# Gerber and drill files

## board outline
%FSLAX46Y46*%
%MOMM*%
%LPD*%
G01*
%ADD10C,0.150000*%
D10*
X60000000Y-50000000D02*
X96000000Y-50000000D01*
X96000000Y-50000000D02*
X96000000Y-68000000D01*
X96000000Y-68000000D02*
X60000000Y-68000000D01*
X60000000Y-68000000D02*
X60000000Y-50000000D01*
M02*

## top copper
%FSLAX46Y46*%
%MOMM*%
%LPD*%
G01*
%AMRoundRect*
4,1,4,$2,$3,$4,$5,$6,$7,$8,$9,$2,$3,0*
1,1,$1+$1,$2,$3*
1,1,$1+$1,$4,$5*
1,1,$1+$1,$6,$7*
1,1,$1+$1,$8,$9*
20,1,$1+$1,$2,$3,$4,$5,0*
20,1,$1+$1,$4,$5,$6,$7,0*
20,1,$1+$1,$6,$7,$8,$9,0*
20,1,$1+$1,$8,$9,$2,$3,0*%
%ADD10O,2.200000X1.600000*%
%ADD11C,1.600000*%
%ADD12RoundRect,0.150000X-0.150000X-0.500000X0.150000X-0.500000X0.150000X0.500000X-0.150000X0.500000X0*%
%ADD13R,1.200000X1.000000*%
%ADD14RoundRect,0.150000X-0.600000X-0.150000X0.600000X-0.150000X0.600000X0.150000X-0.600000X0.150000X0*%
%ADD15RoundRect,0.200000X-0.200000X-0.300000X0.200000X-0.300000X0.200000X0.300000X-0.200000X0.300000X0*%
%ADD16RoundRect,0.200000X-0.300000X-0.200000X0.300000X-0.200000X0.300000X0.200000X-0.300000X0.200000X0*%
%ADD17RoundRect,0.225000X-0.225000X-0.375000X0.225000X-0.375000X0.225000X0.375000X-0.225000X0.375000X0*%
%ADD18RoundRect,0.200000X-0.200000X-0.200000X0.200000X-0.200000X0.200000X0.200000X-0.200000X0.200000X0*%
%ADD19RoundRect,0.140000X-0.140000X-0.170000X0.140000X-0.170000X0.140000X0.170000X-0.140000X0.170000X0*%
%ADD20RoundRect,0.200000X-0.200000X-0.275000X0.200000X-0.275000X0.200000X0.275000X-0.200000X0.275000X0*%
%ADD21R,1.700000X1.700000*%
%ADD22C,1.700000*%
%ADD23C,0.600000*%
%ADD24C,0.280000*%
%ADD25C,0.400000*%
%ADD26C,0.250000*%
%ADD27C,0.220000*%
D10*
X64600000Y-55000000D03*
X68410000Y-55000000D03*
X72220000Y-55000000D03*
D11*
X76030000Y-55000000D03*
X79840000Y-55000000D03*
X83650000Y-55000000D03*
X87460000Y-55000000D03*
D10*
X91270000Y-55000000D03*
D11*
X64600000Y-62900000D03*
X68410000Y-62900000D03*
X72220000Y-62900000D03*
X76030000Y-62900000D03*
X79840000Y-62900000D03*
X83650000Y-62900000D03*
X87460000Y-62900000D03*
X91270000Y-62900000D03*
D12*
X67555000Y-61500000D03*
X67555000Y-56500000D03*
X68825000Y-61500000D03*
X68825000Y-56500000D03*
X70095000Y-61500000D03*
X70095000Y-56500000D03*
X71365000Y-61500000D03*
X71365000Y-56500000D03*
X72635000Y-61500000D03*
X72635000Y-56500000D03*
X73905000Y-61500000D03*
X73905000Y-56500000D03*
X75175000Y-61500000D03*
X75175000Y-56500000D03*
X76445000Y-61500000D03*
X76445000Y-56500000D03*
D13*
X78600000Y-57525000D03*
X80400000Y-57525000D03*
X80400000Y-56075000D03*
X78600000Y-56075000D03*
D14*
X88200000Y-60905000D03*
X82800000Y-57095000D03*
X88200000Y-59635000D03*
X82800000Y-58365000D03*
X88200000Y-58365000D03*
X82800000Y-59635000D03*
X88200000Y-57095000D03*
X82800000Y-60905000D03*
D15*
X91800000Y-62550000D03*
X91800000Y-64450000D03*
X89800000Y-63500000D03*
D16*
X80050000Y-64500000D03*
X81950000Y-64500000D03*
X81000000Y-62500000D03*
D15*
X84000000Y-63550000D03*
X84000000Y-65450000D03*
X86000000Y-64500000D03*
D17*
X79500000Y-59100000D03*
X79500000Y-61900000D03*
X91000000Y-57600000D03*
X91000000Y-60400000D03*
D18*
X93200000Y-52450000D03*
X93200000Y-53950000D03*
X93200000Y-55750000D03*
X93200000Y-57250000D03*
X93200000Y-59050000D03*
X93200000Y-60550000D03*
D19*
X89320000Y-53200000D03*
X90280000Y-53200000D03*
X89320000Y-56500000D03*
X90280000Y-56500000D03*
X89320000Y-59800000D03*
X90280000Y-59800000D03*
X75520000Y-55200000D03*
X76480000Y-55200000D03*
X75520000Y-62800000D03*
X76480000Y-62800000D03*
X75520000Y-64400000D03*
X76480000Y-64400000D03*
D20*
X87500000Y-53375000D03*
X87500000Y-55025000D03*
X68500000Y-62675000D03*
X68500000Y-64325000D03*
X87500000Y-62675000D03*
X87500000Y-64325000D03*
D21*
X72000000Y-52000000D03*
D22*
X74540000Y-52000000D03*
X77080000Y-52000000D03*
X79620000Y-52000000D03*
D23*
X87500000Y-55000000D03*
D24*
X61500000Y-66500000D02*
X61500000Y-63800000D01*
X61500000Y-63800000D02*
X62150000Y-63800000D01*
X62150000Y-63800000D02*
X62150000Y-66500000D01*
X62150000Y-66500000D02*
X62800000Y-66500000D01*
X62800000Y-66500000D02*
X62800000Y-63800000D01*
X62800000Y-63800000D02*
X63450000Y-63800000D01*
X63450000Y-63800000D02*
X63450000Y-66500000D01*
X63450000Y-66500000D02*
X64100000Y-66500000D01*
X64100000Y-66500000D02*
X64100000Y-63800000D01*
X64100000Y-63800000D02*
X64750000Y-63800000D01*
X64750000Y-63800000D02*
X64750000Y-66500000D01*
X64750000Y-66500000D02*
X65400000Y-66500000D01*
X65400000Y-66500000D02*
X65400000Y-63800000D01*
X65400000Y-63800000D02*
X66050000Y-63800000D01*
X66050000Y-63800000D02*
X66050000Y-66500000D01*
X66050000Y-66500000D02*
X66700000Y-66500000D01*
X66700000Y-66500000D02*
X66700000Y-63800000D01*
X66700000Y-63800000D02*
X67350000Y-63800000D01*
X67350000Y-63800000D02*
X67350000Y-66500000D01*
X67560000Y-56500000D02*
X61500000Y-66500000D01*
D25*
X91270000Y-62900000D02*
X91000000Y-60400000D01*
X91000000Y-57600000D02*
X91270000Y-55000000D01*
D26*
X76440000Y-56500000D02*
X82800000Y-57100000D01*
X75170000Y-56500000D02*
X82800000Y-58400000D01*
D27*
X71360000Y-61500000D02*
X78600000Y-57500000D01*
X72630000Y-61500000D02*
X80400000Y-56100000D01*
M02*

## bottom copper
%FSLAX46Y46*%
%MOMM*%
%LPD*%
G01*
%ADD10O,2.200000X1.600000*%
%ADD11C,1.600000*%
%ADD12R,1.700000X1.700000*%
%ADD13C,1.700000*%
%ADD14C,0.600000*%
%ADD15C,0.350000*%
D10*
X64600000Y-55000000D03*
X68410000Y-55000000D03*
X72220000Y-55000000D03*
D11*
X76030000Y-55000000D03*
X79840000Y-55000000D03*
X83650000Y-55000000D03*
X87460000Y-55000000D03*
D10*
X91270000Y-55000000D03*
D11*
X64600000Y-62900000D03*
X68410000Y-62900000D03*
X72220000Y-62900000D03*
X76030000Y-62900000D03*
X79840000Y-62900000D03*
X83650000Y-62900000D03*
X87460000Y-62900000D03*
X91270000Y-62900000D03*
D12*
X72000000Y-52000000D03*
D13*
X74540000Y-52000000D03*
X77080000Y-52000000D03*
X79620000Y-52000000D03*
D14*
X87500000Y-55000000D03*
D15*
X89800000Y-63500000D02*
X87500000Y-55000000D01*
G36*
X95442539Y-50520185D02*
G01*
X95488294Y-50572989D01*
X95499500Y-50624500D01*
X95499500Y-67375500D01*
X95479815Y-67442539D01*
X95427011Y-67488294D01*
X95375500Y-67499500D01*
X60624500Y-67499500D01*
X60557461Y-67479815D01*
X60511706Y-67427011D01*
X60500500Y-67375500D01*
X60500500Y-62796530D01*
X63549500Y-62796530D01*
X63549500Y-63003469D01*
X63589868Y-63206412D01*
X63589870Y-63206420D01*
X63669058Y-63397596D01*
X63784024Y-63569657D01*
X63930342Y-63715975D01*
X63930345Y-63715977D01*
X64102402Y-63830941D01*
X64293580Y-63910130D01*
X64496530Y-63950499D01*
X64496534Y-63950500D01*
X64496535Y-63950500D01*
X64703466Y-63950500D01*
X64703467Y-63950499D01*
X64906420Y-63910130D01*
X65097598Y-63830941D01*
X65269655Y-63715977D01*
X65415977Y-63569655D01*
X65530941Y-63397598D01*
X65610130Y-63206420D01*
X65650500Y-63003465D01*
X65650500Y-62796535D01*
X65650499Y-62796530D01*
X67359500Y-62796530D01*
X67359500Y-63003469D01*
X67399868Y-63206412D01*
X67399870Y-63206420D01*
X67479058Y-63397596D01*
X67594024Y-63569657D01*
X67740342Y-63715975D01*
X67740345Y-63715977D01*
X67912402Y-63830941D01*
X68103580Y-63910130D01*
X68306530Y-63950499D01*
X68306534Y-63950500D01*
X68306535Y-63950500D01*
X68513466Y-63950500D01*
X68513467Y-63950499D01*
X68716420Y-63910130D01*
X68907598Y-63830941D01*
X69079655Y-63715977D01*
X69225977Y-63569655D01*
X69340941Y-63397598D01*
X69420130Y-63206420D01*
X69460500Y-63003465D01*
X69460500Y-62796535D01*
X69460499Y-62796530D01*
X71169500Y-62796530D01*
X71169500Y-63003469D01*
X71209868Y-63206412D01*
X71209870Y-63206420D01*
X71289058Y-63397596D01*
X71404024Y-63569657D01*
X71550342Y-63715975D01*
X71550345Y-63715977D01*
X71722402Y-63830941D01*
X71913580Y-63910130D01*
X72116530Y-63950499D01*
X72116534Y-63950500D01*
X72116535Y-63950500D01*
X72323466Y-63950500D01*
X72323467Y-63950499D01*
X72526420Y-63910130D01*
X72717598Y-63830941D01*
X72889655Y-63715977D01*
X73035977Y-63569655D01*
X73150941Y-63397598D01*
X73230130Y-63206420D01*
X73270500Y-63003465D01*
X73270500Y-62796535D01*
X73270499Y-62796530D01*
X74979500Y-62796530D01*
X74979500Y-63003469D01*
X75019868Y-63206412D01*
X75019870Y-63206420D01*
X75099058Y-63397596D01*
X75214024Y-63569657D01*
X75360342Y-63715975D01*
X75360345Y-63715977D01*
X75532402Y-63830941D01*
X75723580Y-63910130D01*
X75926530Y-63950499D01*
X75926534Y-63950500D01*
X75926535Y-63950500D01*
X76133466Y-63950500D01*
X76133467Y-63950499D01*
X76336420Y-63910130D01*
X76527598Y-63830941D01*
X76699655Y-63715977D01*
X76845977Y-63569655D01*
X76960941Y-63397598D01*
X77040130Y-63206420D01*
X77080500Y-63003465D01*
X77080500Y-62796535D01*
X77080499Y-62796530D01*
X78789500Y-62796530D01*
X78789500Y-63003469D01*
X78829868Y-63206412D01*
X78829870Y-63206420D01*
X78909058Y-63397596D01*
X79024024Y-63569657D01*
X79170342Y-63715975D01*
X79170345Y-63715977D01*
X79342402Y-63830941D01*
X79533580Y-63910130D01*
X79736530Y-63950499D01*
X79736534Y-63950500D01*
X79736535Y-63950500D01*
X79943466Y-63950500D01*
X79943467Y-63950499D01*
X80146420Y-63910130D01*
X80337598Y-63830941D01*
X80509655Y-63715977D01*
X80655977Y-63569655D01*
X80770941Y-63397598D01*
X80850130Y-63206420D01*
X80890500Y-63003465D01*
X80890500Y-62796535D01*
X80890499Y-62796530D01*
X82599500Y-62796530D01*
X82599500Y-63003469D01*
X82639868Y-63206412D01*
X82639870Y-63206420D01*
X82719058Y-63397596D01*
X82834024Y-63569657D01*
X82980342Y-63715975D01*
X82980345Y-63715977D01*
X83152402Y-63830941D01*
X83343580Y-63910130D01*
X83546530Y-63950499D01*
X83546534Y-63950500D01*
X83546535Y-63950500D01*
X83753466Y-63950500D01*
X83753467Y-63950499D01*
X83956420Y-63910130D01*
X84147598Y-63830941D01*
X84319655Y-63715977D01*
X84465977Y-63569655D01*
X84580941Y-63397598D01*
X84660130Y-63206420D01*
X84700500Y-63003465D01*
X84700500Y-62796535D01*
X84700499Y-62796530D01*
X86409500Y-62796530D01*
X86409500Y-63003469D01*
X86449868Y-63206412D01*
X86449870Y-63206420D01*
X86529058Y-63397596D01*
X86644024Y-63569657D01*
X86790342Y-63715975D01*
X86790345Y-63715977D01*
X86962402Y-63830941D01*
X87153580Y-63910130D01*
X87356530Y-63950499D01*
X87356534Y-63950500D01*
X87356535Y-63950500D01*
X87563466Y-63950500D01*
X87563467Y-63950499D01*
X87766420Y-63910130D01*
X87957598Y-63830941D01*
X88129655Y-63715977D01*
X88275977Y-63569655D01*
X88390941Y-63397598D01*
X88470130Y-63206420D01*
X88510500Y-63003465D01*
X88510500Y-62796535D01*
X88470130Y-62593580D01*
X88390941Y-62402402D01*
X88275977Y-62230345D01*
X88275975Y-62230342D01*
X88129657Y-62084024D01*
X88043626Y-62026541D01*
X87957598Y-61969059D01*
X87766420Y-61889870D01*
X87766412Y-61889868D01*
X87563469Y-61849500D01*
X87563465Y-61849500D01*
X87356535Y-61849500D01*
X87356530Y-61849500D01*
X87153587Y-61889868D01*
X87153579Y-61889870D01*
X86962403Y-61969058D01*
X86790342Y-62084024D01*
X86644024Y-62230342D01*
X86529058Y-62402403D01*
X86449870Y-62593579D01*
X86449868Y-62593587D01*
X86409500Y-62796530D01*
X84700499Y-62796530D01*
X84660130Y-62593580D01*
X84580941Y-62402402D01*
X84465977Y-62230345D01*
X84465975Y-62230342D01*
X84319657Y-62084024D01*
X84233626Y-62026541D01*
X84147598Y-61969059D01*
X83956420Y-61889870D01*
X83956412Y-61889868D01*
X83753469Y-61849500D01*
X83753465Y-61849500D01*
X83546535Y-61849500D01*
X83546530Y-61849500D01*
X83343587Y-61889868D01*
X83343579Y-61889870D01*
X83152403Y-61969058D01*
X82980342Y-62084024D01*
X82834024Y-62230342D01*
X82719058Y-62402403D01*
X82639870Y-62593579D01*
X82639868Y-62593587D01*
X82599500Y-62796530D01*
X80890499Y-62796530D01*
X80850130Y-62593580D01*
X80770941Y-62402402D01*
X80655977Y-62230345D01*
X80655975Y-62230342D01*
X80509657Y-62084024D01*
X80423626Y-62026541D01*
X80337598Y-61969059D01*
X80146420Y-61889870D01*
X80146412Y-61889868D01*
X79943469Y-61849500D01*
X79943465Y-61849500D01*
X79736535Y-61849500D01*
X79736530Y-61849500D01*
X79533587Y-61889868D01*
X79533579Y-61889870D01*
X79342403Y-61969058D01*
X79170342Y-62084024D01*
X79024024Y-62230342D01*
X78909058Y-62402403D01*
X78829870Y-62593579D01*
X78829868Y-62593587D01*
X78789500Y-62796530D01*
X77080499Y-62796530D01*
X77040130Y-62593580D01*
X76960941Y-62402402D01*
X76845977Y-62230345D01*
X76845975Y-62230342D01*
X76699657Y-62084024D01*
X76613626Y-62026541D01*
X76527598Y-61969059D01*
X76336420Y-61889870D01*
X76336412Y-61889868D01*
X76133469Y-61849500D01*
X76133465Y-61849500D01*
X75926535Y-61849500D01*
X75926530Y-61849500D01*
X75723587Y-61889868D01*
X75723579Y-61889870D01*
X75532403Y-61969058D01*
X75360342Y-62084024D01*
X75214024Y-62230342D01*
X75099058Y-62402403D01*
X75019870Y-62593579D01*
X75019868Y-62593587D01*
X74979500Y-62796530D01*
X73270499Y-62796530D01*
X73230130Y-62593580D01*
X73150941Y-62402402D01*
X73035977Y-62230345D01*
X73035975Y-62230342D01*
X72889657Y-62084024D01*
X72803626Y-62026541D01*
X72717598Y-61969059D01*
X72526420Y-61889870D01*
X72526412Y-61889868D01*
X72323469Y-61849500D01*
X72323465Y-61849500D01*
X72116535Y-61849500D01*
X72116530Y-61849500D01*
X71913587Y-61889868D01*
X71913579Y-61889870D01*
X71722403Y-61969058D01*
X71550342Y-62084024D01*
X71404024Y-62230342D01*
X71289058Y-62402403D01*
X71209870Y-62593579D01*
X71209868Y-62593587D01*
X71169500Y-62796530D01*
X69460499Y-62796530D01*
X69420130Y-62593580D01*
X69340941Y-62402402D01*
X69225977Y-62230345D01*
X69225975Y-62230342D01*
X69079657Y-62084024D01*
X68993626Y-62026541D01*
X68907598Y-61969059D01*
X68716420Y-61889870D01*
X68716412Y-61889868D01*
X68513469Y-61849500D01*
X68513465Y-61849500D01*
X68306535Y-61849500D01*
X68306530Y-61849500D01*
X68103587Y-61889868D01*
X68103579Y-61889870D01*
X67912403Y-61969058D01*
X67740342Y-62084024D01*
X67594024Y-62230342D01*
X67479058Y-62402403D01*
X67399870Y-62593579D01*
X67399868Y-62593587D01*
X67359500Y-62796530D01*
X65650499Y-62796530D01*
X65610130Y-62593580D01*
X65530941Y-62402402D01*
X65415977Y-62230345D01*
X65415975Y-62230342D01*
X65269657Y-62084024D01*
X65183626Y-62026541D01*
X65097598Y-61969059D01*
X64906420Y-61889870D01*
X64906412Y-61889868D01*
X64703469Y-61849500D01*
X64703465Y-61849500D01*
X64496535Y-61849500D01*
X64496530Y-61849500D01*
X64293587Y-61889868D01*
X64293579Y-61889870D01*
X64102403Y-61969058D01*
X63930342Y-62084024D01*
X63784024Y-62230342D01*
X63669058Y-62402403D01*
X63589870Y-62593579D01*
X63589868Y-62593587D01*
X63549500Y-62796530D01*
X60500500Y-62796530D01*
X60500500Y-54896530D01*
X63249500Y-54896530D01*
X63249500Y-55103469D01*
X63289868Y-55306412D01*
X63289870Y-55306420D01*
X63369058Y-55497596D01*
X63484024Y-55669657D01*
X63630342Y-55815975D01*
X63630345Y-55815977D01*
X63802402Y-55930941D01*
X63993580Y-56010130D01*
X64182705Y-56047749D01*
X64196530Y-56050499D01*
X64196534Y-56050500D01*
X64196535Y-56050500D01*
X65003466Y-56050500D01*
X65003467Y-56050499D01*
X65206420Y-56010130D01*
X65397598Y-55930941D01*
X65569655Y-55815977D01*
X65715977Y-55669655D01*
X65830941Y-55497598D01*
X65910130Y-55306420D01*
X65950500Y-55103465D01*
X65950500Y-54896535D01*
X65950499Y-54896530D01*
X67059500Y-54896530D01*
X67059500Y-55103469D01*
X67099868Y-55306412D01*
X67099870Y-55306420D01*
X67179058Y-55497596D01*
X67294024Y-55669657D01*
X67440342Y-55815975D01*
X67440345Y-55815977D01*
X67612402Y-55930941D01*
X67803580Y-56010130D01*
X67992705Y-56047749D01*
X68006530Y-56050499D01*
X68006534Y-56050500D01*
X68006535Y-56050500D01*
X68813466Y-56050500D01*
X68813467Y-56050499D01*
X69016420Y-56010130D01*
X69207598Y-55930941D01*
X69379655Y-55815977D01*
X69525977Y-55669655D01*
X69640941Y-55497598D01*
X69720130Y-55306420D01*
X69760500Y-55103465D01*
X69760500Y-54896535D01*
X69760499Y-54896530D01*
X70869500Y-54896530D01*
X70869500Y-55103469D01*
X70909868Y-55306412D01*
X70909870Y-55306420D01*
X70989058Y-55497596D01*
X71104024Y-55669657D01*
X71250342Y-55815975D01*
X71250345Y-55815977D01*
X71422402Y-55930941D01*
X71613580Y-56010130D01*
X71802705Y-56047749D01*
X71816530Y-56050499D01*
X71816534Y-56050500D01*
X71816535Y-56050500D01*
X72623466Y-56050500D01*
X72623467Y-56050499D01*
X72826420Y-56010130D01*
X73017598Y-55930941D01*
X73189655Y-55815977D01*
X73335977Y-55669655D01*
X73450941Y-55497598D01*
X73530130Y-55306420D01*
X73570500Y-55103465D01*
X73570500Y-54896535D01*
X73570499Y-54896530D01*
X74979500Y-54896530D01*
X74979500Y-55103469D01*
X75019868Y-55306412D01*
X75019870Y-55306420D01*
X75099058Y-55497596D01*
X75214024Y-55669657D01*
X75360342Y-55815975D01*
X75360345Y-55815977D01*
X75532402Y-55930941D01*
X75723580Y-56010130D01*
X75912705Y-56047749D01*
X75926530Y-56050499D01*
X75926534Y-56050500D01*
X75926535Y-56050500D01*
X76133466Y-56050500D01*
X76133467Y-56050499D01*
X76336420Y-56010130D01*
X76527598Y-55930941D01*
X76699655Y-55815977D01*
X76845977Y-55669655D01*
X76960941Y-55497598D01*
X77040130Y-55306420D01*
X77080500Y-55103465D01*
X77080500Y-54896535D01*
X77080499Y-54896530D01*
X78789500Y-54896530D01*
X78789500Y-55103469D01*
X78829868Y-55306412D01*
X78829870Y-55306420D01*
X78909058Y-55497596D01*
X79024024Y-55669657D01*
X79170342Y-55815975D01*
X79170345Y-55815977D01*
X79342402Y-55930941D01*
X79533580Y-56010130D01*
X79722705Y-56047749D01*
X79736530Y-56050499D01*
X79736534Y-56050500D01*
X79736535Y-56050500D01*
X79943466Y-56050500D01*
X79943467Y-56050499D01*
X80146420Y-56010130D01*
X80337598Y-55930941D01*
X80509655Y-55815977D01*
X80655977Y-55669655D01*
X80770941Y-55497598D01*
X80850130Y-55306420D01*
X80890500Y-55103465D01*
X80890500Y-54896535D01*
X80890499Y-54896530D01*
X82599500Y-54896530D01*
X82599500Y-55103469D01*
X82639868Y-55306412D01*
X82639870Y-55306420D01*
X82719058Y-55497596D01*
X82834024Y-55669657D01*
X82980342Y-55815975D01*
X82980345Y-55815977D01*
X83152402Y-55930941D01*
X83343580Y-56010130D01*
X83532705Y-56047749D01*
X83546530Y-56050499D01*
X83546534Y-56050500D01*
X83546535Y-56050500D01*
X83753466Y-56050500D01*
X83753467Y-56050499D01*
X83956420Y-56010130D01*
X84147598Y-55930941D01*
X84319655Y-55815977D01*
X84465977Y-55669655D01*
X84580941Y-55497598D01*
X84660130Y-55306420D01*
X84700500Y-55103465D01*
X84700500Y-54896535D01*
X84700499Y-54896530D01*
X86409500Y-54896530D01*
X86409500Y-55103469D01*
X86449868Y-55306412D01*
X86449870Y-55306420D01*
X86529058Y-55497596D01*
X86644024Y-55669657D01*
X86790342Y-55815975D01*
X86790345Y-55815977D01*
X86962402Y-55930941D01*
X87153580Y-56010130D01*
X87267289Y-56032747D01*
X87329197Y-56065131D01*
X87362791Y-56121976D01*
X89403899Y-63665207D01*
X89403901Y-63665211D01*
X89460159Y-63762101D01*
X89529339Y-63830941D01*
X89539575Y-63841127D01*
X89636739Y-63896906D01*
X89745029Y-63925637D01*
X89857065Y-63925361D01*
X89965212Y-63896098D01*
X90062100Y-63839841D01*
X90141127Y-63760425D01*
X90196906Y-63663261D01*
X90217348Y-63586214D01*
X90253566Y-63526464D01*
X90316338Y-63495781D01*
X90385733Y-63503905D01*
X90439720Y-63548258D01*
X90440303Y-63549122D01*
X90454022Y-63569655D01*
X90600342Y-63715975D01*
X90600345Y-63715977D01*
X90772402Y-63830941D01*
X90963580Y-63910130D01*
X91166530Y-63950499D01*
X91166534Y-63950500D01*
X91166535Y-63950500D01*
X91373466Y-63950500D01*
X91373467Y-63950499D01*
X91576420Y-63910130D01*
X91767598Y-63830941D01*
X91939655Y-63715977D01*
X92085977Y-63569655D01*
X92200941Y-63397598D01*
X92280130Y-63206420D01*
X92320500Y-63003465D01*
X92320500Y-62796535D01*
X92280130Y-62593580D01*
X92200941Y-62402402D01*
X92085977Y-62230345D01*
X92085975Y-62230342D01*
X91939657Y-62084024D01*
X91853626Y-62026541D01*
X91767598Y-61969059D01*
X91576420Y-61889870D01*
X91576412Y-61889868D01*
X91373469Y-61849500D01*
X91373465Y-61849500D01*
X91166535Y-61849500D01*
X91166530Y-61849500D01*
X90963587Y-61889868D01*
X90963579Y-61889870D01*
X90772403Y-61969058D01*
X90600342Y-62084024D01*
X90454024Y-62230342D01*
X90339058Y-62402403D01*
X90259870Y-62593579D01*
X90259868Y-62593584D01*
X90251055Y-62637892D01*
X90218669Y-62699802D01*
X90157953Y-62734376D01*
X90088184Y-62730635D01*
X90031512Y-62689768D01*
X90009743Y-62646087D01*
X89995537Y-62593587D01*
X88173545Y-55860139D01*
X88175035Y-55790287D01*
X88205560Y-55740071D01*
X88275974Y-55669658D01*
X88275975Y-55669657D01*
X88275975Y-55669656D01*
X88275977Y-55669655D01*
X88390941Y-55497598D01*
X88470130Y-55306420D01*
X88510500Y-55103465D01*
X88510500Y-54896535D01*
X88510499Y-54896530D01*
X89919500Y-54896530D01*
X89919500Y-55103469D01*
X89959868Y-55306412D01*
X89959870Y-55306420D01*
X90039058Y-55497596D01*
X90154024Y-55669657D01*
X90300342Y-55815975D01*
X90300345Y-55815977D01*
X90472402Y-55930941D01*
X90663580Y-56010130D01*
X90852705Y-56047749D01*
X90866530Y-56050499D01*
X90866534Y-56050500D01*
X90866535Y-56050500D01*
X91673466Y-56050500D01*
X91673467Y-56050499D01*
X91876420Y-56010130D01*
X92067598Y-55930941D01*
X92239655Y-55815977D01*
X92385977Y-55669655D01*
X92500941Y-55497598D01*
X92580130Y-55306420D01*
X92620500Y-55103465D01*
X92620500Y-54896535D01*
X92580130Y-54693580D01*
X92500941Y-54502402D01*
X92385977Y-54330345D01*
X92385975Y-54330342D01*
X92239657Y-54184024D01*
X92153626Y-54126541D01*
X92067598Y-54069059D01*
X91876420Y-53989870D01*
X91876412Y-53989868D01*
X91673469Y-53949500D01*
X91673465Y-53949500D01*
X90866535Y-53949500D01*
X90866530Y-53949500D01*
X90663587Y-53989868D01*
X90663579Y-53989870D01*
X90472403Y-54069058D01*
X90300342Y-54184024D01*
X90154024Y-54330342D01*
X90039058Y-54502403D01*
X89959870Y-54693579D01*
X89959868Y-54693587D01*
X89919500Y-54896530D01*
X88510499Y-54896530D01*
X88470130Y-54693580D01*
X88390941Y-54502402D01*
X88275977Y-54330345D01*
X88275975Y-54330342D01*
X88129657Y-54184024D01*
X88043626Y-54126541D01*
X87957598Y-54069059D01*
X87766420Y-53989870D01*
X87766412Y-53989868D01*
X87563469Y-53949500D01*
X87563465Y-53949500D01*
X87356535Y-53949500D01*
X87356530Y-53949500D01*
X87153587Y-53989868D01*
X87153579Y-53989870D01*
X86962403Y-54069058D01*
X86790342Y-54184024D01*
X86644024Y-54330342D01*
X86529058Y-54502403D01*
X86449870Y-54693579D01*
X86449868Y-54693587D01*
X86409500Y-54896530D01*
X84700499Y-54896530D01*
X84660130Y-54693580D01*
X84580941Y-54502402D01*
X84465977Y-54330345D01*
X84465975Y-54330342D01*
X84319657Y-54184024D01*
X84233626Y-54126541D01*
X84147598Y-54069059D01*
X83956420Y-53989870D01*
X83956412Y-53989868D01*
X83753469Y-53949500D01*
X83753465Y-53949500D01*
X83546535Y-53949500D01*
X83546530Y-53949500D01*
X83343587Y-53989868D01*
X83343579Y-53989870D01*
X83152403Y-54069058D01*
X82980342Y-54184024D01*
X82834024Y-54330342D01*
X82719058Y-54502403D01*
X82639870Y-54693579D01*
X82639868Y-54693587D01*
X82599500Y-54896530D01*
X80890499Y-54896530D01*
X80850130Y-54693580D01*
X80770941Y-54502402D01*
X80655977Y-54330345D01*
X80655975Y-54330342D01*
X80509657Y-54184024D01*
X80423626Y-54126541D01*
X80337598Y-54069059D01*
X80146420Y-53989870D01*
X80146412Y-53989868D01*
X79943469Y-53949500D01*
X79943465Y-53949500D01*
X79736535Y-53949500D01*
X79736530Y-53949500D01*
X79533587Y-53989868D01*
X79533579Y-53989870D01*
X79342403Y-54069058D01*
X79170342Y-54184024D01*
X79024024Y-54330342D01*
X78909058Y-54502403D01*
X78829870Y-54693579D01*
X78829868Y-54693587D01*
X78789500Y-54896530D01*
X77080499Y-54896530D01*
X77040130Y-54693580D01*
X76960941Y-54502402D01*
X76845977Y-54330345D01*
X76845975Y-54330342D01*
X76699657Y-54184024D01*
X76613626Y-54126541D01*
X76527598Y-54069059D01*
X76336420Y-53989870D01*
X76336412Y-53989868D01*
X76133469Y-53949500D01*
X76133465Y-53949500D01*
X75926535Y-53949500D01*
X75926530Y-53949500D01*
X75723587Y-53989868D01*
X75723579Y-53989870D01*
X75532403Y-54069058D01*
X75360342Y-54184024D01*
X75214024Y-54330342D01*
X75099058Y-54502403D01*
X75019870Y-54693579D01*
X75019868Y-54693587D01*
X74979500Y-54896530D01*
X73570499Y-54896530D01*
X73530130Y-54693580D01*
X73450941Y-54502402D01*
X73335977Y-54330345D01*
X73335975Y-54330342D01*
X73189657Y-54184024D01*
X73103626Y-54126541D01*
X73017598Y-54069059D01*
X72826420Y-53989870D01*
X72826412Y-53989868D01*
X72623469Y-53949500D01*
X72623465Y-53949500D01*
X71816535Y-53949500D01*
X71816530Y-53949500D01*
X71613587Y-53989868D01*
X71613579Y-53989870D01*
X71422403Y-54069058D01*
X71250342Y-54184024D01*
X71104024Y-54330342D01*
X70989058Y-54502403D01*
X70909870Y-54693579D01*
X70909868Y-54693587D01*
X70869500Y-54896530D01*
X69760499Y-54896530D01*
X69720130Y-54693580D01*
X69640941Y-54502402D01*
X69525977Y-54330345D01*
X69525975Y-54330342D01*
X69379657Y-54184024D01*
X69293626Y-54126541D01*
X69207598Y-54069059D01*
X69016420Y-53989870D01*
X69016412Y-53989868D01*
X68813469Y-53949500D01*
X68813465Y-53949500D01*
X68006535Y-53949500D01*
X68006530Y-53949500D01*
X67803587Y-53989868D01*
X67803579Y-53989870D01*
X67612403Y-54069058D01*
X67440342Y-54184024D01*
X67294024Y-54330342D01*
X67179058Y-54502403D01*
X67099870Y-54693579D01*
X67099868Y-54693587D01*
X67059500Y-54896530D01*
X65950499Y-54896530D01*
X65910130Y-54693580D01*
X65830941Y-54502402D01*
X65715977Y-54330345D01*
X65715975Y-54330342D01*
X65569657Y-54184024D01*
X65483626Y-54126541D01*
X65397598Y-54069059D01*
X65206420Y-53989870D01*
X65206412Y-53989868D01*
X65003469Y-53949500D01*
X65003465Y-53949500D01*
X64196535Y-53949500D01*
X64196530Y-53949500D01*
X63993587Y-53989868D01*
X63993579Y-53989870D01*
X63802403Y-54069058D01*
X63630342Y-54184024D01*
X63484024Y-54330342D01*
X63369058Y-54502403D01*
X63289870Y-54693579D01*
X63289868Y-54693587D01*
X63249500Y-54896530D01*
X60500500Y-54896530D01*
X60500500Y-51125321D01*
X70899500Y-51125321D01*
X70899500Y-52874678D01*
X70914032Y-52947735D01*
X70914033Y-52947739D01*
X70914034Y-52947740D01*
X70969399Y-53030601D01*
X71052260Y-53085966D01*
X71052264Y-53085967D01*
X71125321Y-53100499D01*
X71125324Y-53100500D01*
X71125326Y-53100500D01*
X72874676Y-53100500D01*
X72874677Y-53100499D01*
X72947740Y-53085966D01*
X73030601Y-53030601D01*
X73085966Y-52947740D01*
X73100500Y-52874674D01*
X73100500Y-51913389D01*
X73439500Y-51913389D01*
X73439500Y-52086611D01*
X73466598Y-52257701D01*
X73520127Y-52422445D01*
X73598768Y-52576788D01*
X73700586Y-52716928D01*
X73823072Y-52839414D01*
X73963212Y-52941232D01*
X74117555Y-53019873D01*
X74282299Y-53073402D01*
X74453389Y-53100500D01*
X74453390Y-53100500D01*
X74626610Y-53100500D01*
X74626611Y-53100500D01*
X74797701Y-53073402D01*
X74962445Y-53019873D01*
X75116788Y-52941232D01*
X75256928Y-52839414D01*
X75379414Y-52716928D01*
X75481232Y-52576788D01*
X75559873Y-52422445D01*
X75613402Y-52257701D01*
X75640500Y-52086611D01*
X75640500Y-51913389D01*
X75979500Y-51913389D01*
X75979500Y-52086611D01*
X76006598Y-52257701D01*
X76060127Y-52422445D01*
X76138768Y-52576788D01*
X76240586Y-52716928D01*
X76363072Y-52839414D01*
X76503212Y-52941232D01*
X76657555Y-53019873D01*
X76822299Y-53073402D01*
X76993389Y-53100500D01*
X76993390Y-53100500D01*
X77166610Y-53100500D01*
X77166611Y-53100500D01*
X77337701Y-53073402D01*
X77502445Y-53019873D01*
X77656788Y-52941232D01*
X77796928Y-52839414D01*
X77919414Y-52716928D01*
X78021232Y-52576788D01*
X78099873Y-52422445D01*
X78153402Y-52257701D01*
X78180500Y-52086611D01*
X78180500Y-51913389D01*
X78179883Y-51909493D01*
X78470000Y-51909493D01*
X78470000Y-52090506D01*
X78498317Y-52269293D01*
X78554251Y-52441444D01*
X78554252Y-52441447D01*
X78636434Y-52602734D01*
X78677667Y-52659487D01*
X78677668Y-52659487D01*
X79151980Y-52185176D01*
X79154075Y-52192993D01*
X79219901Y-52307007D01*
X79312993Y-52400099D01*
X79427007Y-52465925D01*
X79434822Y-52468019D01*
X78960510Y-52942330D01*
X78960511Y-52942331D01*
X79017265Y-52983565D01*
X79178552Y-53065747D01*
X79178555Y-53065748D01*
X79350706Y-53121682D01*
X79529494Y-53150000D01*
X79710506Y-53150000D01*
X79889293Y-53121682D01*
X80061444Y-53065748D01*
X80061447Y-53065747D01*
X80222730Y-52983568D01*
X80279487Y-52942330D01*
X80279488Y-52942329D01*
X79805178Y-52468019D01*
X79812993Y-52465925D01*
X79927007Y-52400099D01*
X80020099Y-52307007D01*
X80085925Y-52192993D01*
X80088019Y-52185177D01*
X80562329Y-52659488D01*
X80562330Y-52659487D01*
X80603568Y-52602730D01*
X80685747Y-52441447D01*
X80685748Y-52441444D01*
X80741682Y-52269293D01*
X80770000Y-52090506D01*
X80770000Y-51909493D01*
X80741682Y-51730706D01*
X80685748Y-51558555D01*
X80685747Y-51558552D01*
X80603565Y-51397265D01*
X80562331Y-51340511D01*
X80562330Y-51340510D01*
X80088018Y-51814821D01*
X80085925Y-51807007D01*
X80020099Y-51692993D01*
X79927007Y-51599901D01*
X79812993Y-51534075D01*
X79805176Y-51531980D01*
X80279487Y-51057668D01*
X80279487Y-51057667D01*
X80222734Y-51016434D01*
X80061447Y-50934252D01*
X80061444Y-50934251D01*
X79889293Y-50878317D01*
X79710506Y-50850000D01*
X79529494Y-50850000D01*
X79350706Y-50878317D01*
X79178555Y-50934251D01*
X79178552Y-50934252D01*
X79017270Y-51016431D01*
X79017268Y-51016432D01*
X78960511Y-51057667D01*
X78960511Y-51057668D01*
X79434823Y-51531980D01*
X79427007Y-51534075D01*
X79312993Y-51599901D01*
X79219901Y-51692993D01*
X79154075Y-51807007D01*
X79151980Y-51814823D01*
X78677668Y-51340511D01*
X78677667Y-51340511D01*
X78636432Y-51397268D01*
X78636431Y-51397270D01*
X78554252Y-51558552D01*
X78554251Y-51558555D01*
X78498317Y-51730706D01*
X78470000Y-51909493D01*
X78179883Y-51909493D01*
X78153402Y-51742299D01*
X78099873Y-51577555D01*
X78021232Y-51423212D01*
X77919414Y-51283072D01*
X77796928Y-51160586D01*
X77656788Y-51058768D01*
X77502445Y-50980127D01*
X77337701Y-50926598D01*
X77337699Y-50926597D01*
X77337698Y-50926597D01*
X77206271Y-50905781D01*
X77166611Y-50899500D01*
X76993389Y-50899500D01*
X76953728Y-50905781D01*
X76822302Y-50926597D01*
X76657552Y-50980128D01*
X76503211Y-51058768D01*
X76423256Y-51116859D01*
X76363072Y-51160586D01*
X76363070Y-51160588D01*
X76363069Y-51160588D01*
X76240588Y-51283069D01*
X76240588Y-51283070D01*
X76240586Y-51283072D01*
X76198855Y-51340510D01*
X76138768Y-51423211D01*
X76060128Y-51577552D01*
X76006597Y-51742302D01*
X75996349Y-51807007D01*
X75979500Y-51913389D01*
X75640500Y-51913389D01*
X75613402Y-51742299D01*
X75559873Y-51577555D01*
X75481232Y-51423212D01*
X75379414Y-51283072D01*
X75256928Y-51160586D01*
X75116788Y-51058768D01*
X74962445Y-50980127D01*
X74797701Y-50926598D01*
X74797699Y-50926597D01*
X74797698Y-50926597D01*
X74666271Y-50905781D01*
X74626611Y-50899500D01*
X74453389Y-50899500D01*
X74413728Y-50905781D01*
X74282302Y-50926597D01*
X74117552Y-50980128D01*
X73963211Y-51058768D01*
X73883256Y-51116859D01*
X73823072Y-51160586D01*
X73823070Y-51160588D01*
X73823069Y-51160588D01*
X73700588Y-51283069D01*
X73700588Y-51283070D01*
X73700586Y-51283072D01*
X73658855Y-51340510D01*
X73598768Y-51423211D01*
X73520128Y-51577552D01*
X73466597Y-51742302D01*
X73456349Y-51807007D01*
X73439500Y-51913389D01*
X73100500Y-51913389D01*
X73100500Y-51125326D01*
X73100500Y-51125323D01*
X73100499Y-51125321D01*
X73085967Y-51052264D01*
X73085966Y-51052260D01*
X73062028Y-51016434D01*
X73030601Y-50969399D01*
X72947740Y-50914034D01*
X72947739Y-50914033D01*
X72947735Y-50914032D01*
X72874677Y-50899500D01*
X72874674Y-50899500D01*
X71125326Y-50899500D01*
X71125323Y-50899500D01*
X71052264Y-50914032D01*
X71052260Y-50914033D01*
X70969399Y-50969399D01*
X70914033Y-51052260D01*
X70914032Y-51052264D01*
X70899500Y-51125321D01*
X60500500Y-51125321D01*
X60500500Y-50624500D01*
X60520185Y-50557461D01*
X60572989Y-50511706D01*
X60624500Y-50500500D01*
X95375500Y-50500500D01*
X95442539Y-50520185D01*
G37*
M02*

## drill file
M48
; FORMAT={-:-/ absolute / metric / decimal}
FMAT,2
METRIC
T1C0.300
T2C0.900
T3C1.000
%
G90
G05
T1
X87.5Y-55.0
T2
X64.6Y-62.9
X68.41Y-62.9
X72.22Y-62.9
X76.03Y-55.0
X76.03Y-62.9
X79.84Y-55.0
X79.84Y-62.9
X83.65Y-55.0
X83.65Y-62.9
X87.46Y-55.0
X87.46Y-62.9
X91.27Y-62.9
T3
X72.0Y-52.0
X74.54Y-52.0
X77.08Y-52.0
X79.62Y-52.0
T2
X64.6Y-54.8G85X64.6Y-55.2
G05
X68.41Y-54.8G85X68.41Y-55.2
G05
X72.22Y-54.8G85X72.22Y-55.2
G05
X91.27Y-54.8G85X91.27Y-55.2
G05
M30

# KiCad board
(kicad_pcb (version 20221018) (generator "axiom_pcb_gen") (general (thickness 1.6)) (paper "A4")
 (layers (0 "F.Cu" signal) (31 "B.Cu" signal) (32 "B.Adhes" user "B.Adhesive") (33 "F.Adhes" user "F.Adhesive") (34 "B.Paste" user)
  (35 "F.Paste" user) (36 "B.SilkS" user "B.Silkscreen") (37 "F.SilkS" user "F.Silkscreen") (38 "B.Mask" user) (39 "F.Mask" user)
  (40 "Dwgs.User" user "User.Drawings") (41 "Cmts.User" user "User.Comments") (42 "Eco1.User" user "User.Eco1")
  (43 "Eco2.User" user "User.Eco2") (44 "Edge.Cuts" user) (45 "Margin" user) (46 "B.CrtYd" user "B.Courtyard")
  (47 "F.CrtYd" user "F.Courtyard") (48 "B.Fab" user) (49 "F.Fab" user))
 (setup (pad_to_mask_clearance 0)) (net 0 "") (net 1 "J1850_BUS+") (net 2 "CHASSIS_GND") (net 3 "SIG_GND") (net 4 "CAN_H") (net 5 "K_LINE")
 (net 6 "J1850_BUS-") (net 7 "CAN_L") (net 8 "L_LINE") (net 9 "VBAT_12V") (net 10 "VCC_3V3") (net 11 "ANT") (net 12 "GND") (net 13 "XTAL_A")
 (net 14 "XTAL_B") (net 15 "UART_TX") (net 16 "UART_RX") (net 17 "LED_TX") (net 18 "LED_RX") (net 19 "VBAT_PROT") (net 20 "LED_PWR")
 (gr_line (start 60.000 50.000) (end 96.000 50.000) (stroke (width 0.15) (type default)) (layer "Edge.Cuts"))
 (gr_line (start 96.000 50.000) (end 96.000 68.000) (stroke (width 0.15) (type default)) (layer "Edge.Cuts"))
 (gr_line (start 96.000 68.000) (end 60.000 68.000) (stroke (width 0.15) (type default)) (layer "Edge.Cuts"))
 (gr_line (start 60.000 68.000) (end 60.000 50.000) (stroke (width 0.15) (type default)) (layer "Edge.Cuts"))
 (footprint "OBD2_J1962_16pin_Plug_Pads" (layer "F.Cu") (at 64.600 55.000)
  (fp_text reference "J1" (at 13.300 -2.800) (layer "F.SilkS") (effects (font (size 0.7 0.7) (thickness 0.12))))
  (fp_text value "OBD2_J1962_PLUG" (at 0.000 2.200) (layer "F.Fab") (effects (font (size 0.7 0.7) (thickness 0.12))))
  (pad "1" thru_hole oval (at 0.000 0.000) (size 2.2 1.6) (drill oval 0.9 1.3) (layers "*.Cu" "*.Mask"))
  (pad "2" thru_hole oval (at 3.810 0.000) (size 2.2 1.6) (drill oval 0.9 1.3) (layers "*.Cu" "*.Mask") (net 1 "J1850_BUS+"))
  (pad "3" thru_hole oval (at 7.620 0.000) (size 2.2 1.6) (drill oval 0.9 1.3) (layers "*.Cu" "*.Mask"))
  (pad "4" thru_hole circle (at 11.430 0.000) (size 1.6 1.6) (drill 0.9) (layers "*.Cu" "*.Mask") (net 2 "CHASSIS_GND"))
  (pad "5" thru_hole circle (at 15.240 0.000) (size 1.6 1.6) (drill 0.9) (layers "*.Cu" "*.Mask") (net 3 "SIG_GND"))
  (pad "6" thru_hole circle (at 19.050 0.000) (size 1.6 1.6) (drill 0.9) (layers "*.Cu" "*.Mask") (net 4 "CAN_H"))
  (pad "7" thru_hole circle (at 22.860 0.000) (size 1.6 1.6) (drill 0.9) (layers "*.Cu" "*.Mask") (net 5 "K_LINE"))
  (pad "8" thru_hole oval (at 26.670 0.000) (size 2.2 1.6) (drill oval 0.9 1.3) (layers "*.Cu" "*.Mask"))
  (pad "9" thru_hole circle (at 0.000 7.900) (size 1.6 1.6) (drill 0.9) (layers "*.Cu" "*.Mask"))
  (pad "10" thru_hole circle (at 3.810 7.900) (size 1.6 1.6) (drill 0.9) (layers "*.Cu" "*.Mask") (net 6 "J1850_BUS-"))
  (pad "11" thru_hole circle (at 7.620 7.900) (size 1.6 1.6) (drill 0.9) (layers "*.Cu" "*.Mask"))
  (pad "12" thru_hole circle (at 11.430 7.900) (size 1.6 1.6) (drill 0.9) (layers "*.Cu" "*.Mask"))
  (pad "13" thru_hole circle (at 15.240 7.900) (size 1.6 1.6) (drill 0.9) (layers "*.Cu" "*.Mask"))
  (pad "14" thru_hole circle (at 19.050 7.900) (size 1.6 1.6) (drill 0.9) (layers "*.Cu" "*.Mask") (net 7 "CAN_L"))
  (pad "15" thru_hole circle (at 22.860 7.900) (size 1.6 1.6) (drill 0.9) (layers "*.Cu" "*.Mask") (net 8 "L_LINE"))
  (pad "16" thru_hole circle (at 26.670 7.900) (size 1.6 1.6) (drill 0.9) (layers "*.Cu" "*.Mask") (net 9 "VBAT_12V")))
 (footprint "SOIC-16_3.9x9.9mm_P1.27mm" (layer "F.Cu") (at 72.000 59.000)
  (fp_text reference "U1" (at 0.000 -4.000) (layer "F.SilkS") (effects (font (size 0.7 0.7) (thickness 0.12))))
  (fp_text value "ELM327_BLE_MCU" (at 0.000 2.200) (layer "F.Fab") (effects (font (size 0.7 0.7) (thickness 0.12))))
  (pad "1" smd roundrect (at -4.445 2.500) (size 0.6 1.3) (layers "F.Cu" "F.Paste" "F.Mask") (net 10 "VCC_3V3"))
  (pad "16" smd roundrect (at -4.445 -2.500) (size 0.6 1.3) (layers "F.Cu" "F.Paste" "F.Mask") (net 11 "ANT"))
  (pad "2" smd roundrect (at -3.175 2.500) (size 0.6 1.3) (layers "F.Cu" "F.Paste" "F.Mask") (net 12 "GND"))
  (pad "15" smd roundrect (at -3.175 -2.500) (size 0.6 1.3) (layers "F.Cu" "F.Paste" "F.Mask"))
  (pad "3" smd roundrect (at -1.905 2.500) (size 0.6 1.3) (layers "F.Cu" "F.Paste" "F.Mask") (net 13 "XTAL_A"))
  (pad "14" smd roundrect (at -1.905 -2.500) (size 0.6 1.3) (layers "F.Cu" "F.Paste" "F.Mask"))
  (pad "4" smd roundrect (at -0.635 2.500) (size 0.6 1.3) (layers "F.Cu" "F.Paste" "F.Mask") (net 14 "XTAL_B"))
  (pad "13" smd roundrect (at -0.635 -2.500) (size 0.6 1.3) (layers "F.Cu" "F.Paste" "F.Mask") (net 4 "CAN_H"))
  (pad "5" smd roundrect (at 0.635 2.500) (size 0.6 1.3) (layers "F.Cu" "F.Paste" "F.Mask") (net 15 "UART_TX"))
  (pad "12" smd roundrect (at 0.635 -2.500) (size 0.6 1.3) (layers "F.Cu" "F.Paste" "F.Mask") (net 7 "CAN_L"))
  (pad "6" smd roundrect (at 1.905 2.500) (size 0.6 1.3) (layers "F.Cu" "F.Paste" "F.Mask") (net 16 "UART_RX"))
  (pad "11" smd roundrect (at 1.905 -2.500) (size 0.6 1.3) (layers "F.Cu" "F.Paste" "F.Mask") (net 5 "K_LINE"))
  (pad "7" smd roundrect (at 3.175 2.500) (size 0.6 1.3) (layers "F.Cu" "F.Paste" "F.Mask") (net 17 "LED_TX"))
  (pad "10" smd roundrect (at 3.175 -2.500) (size 0.6 1.3) (layers "F.Cu" "F.Paste" "F.Mask") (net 8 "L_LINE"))
  (pad "8" smd roundrect (at 4.445 2.500) (size 0.6 1.3) (layers "F.Cu" "F.Paste" "F.Mask") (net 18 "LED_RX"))
  (pad "9" smd roundrect (at 4.445 -2.500) (size 0.6 1.3) (layers "F.Cu" "F.Paste" "F.Mask") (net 12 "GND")))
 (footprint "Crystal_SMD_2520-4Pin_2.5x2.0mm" (layer "F.Cu") (at 79.500 56.800)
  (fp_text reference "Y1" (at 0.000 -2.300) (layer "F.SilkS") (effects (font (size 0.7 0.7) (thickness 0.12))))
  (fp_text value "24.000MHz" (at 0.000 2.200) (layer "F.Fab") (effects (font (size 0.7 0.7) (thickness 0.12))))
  (pad "1" smd rect (at -0.900 0.725) (size 1.2 1.0) (layers "F.Cu" "F.Paste" "F.Mask") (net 13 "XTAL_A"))
  (pad "2" smd rect (at 0.900 0.725) (size 1.2 1.0) (layers "F.Cu" "F.Paste" "F.Mask") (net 12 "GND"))
  (pad "3" smd rect (at 0.900 -0.725) (size 1.2 1.0) (layers "F.Cu" "F.Paste" "F.Mask") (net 14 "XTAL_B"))
  (pad "4" smd rect (at -0.900 -0.725) (size 1.2 1.0) (layers "F.Cu" "F.Paste" "F.Mask") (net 12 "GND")))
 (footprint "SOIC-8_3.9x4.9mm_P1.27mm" (layer "F.Cu") (at 85.500 59.000)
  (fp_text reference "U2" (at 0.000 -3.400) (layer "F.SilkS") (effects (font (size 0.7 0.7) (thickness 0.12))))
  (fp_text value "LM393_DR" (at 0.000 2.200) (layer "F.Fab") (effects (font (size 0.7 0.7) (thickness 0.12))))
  (pad "1" smd roundrect (at 2.700 1.905) (size 1.5 0.6) (layers "F.Cu" "F.Paste" "F.Mask") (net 5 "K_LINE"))
  (pad "5" smd roundrect (at -2.700 -1.905) (size 1.5 0.6) (layers "F.Cu" "F.Paste" "F.Mask") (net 8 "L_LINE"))
  (pad "2" smd roundrect (at 2.700 0.635) (size 1.5 0.6) (layers "F.Cu" "F.Paste" "F.Mask") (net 5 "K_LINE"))
  (pad "6" smd roundrect (at -2.700 -0.635) (size 1.5 0.6) (layers "F.Cu" "F.Paste" "F.Mask") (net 8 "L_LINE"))
  (pad "3" smd roundrect (at 2.700 -0.635) (size 1.5 0.6) (layers "F.Cu" "F.Paste" "F.Mask") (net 5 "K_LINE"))
  (pad "7" smd roundrect (at -2.700 0.635) (size 1.5 0.6) (layers "F.Cu" "F.Paste" "F.Mask") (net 8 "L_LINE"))
  (pad "4" smd roundrect (at 2.700 -1.905) (size 1.5 0.6) (layers "F.Cu" "F.Paste" "F.Mask") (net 12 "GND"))
  (pad "8" smd roundrect (at -2.700 1.905) (size 1.5 0.6) (layers "F.Cu" "F.Paste" "F.Mask") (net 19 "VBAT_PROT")))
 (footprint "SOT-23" (layer "F.Cu") (at 90.800 63.500)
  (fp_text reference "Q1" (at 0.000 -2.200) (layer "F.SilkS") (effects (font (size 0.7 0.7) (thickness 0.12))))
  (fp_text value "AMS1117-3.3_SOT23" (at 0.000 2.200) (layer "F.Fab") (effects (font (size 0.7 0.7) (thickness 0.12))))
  (pad "1" smd roundrect (at 1.000 -0.950) (size 0.8 1.0) (layers "F.Cu" "F.Paste" "F.Mask") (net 12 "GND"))
  (pad "2" smd roundrect (at 1.000 0.950) (size 0.8 1.0) (layers "F.Cu" "F.Paste" "F.Mask") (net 19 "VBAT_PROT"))
  (pad "3" smd roundrect (at -1.000 0.000) (size 0.8 1.0) (layers "F.Cu" "F.Paste" "F.Mask") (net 10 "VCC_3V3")))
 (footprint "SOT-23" (layer "F.Cu") (at 81.000 63.500)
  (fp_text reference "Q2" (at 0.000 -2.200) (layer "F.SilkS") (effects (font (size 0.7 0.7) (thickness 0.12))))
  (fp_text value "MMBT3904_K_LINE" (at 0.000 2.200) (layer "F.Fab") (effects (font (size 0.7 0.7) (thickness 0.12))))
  (pad "1" smd roundrect (at -0.950 1.000) (size 1.0 0.8) (layers "F.Cu" "F.Paste" "F.Mask") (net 5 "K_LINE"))
  (pad "2" smd roundrect (at 0.950 1.000) (size 1.0 0.8) (layers "F.Cu" "F.Paste" "F.Mask") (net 12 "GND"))
  (pad "3" smd roundrect (at 0.000 -1.000) (size 1.0 0.8) (layers "F.Cu" "F.Paste" "F.Mask") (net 15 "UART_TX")))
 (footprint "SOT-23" (layer "F.Cu") (at 85.000 64.500)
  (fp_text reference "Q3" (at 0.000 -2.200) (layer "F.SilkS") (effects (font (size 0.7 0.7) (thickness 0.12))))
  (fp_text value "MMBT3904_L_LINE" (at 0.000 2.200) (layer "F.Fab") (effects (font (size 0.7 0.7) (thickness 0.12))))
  (pad "1" smd roundrect (at -1.000 -0.950) (size 0.8 1.0) (layers "F.Cu" "F.Paste" "F.Mask") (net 8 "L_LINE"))
  (pad "2" smd roundrect (at -1.000 0.950) (size 0.8 1.0) (layers "F.Cu" "F.Paste" "F.Mask") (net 12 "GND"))
  (pad "3" smd roundrect (at 1.000 0.000) (size 0.8 1.0) (layers "F.Cu" "F.Paste" "F.Mask") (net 16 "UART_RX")))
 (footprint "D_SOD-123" (layer "F.Cu") (at 79.500 60.500)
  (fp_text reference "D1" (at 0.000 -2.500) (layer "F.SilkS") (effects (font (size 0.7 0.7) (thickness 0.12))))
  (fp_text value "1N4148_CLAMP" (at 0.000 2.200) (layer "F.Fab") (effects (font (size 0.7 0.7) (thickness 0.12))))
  (pad "1" smd roundrect (at 0.000 -1.400) (size 0.9 1.2) (layers "F.Cu" "F.Paste" "F.Mask") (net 4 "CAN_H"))
  (pad "2" smd roundrect (at 0.000 1.400) (size 0.9 1.2) (layers "F.Cu" "F.Paste" "F.Mask") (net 12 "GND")))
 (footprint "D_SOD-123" (layer "F.Cu") (at 91.000 59.000)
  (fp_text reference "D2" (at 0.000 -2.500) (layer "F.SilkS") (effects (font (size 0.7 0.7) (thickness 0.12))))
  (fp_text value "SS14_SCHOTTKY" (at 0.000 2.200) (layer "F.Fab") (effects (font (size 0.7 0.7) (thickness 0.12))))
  (pad "1" smd roundrect (at 0.000 -1.400) (size 0.9 1.2) (layers "F.Cu" "F.Paste" "F.Mask") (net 9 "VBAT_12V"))
  (pad "2" smd roundrect (at 0.000 1.400) (size 0.9 1.2) (layers "F.Cu" "F.Paste" "F.Mask") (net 19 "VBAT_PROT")))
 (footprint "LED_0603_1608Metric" (layer "F.Cu") (at 93.200 53.200)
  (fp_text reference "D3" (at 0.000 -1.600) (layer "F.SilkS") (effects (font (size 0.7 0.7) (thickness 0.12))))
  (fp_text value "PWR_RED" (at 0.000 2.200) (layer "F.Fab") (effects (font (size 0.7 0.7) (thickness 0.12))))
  (pad "1" smd roundrect (at 0.000 -0.750) (size 0.8 0.8) (layers "F.Cu" "F.Paste" "F.Mask") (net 10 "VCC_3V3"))
  (pad "2" smd roundrect (at 0.000 0.750) (size 0.8 0.8) (layers "F.Cu" "F.Paste" "F.Mask") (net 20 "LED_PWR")))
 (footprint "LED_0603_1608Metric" (layer "F.Cu") (at 93.200 56.500)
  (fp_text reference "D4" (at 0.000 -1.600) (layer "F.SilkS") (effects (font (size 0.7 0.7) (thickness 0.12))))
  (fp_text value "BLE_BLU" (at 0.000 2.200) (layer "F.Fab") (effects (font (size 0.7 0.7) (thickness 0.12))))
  (pad "1" smd roundrect (at 0.000 -0.750) (size 0.8 0.8) (layers "F.Cu" "F.Paste" "F.Mask") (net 10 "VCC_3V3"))
  (pad "2" smd roundrect (at 0.000 0.750) (size 0.8 0.8) (layers "F.Cu" "F.Paste" "F.Mask") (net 17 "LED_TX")))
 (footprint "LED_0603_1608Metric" (layer "F.Cu") (at 93.200 59.800)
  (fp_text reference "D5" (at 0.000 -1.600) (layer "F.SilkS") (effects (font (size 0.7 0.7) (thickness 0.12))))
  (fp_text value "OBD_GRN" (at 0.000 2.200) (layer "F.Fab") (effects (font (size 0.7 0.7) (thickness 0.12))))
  (pad "1" smd roundrect (at 0.000 -0.750) (size 0.8 0.8) (layers "F.Cu" "F.Paste" "F.Mask") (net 10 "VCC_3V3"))
  (pad "2" smd roundrect (at 0.000 0.750) (size 0.8 0.8) (layers "F.Cu" "F.Paste" "F.Mask") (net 18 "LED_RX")))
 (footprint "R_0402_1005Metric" (layer "F.Cu") (at 89.800 53.200)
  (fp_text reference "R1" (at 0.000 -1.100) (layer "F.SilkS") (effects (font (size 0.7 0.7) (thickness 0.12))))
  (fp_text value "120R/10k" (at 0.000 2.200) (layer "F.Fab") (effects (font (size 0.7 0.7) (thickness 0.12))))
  (pad "1" smd roundrect (at -0.480 0.000) (size 0.56 0.62) (layers "F.Cu" "F.Paste" "F.Mask") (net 20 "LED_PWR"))
  (pad "2" smd roundrect (at 0.480 0.000) (size 0.56 0.62) (layers "F.Cu" "F.Paste" "F.Mask") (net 12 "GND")))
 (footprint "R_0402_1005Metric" (layer "F.Cu") (at 89.800 56.500)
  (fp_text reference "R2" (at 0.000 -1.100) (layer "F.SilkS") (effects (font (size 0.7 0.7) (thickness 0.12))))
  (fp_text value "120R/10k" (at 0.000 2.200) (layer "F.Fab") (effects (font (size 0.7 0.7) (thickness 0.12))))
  (pad "1" smd roundrect (at -0.480 0.000) (size 0.56 0.62) (layers "F.Cu" "F.Paste" "F.Mask") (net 17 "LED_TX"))
  (pad "2" smd roundrect (at 0.480 0.000) (size 0.56 0.62) (layers "F.Cu" "F.Paste" "F.Mask") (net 12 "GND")))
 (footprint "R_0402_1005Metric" (layer "F.Cu") (at 89.800 59.800)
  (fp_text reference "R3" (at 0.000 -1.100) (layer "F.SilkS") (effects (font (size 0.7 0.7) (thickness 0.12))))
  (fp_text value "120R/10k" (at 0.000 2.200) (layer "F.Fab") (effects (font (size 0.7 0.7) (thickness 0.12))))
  (pad "1" smd roundrect (at -0.480 0.000) (size 0.56 0.62) (layers "F.Cu" "F.Paste" "F.Mask") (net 18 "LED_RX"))
  (pad "2" smd roundrect (at 0.480 0.000) (size 0.56 0.62) (layers "F.Cu" "F.Paste" "F.Mask") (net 12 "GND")))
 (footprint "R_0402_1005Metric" (layer "F.Cu") (at 76.000 55.200)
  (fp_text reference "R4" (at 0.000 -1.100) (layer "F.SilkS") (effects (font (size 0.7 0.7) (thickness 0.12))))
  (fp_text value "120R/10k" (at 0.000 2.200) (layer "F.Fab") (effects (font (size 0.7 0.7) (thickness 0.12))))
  (pad "1" smd roundrect (at -0.480 0.000) (size 0.56 0.62) (layers "F.Cu" "F.Paste" "F.Mask") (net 4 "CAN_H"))
  (pad "2" smd roundrect (at 0.480 0.000) (size 0.56 0.62) (layers "F.Cu" "F.Paste" "F.Mask") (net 7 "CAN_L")))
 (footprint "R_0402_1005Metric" (layer "F.Cu") (at 76.000 62.800)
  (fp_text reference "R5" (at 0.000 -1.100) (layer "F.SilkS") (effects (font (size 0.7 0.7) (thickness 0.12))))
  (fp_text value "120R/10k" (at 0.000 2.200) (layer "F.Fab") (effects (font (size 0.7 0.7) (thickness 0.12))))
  (pad "1" smd roundrect (at -0.480 0.000) (size 0.56 0.62) (layers "F.Cu" "F.Paste" "F.Mask") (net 5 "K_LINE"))
  (pad "2" smd roundrect (at 0.480 0.000) (size 0.56 0.62) (layers "F.Cu" "F.Paste" "F.Mask") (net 10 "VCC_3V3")))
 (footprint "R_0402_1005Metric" (layer "F.Cu") (at 76.000 64.400)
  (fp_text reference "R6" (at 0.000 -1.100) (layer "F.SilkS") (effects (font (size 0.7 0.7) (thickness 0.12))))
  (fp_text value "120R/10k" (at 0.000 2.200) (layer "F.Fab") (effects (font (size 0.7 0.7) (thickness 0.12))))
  (pad "1" smd roundrect (at -0.480 0.000) (size 0.56 0.62) (layers "F.Cu" "F.Paste" "F.Mask") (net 8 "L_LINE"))
  (pad "2" smd roundrect (at 0.480 0.000) (size 0.56 0.62) (layers "F.Cu" "F.Paste" "F.Mask") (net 10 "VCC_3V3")))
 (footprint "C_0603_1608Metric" (layer "F.Cu") (at 87.500 54.200)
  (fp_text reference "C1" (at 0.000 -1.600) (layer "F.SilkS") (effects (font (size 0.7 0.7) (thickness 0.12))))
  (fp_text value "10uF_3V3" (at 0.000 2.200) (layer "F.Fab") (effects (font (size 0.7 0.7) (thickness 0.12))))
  (pad "1" smd roundrect (at 0.000 -0.825) (size 0.8 0.95) (layers "F.Cu" "F.Paste" "F.Mask") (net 10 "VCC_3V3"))
  (pad "2" smd roundrect (at 0.000 0.825) (size 0.8 0.95) (layers "F.Cu" "F.Paste" "F.Mask") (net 12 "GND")))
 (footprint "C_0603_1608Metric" (layer "F.Cu") (at 68.500 63.500)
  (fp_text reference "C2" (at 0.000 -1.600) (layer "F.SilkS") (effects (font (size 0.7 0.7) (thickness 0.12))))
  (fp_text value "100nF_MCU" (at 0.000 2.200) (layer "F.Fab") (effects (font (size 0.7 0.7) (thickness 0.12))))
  (pad "1" smd roundrect (at 0.000 -0.825) (size 0.8 0.95) (layers "F.Cu" "F.Paste" "F.Mask") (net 10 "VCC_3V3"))
  (pad "2" smd roundrect (at 0.000 0.825) (size 0.8 0.95) (layers "F.Cu" "F.Paste" "F.Mask") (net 12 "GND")))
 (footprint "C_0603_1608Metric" (layer "F.Cu") (at 87.500 63.500)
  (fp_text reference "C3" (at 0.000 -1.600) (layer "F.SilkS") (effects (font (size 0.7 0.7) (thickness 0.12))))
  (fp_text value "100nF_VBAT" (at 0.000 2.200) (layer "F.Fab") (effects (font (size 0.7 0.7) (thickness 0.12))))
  (pad "1" smd roundrect (at 0.000 -0.825) (size 0.8 0.95) (layers "F.Cu" "F.Paste" "F.Mask") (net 19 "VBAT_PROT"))
  (pad "2" smd roundrect (at 0.000 0.825) (size 0.8 0.95) (layers "F.Cu" "F.Paste" "F.Mask") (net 12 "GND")))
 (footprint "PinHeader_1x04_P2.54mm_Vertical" (layer "F.Cu") (at 72.000 52.000)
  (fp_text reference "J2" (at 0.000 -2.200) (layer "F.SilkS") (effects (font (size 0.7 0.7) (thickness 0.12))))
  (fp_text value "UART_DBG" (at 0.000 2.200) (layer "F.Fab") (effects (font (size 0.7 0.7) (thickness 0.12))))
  (pad "1" thru_hole rect (at 0.000 0.000) (size 1.7 1.7) (drill 1.0) (layers "*.Cu" "*.Mask") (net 10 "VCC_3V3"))
  (pad "2" thru_hole circle (at 2.540 0.000) (size 1.7 1.7) (drill 1.0) (layers "*.Cu" "*.Mask") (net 15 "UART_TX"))
  (pad "3" thru_hole circle (at 5.080 0.000) (size 1.7 1.7) (drill 1.0) (layers "*.Cu" "*.Mask") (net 16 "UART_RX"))
  (pad "4" thru_hole circle (at 7.620 0.000) (size 1.7 1.7) (drill 1.0) (layers "*.Cu" "*.Mask") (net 12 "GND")))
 (segment (start 61.500 66.500) (end 61.500 63.800) (width 0.28) (layer "F.Cu") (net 11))
 (segment (start 61.500 63.800) (end 62.150 63.800) (width 0.28) (layer "F.Cu") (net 11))
 (segment (start 62.150 63.800) (end 62.150 66.500) (width 0.28) (layer "F.Cu") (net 11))
 (segment (start 62.150 66.500) (end 62.800 66.500) (width 0.28) (layer "F.Cu") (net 11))
 (segment (start 62.800 66.500) (end 62.800 63.800) (width 0.28) (layer "F.Cu") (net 11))
 (segment (start 62.800 63.800) (end 63.450 63.800) (width 0.28) (layer "F.Cu") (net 11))
 (segment (start 63.450 63.800) (end 63.450 66.500) (width 0.28) (layer "F.Cu") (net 11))
 (segment (start 63.450 66.500) (end 64.100 66.500) (width 0.28) (layer "F.Cu") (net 11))
 (segment (start 64.100 66.500) (end 64.100 63.800) (width 0.28) (layer "F.Cu") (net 11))
 (segment (start 64.100 63.800) (end 64.750 63.800) (width 0.28) (layer "F.Cu") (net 11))
 (segment (start 64.750 63.800) (end 64.750 66.500) (width 0.28) (layer "F.Cu") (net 11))
 (segment (start 64.750 66.500) (end 65.400 66.500) (width 0.28) (layer "F.Cu") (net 11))
 (segment (start 65.400 66.500) (end 65.400 63.800) (width 0.28) (layer "F.Cu") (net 11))
 (segment (start 65.400 63.800) (end 66.050 63.800) (width 0.28) (layer "F.Cu") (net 11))
 (segment (start 66.050 63.800) (end 66.050 66.500) (width 0.28) (layer "F.Cu") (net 11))
 (segment (start 66.050 66.500) (end 66.700 66.500) (width 0.28) (layer "F.Cu") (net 11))
 (segment (start 66.700 66.500) (end 66.700 63.800) (width 0.28) (layer "F.Cu") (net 11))
 (segment (start 66.700 63.800) (end 67.350 63.800) (width 0.28) (layer "F.Cu") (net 11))
 (segment (start 67.350 63.800) (end 67.350 66.500) (width 0.28) (layer "F.Cu") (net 11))
 (segment (start 67.560 56.500) (end 61.500 66.500) (width 0.28) (layer "F.Cu") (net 11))
 (segment (start 91.270 62.900) (end 91.000 60.400) (width 0.4) (layer "F.Cu") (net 19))
 (segment (start 91.000 57.600) (end 91.270 55.000) (width 0.4) (layer "F.Cu") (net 9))
 (segment (start 89.800 63.500) (end 87.500 55.000) (width 0.35) (layer "B.Cu") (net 10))
 (via (at 87.500 55.000) (size 0.6) (drill 0.3) (layers "F.Cu" "B.Cu") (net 10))
 (segment (start 76.440 56.500) (end 82.800 57.100) (width 0.25) (layer "F.Cu") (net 5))
 (segment (start 75.170 56.500) (end 82.800 58.400) (width 0.25) (layer "F.Cu") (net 8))
 (segment (start 71.360 61.500) (end 78.600 57.500) (width 0.22) (layer "F.Cu") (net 13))
 (segment (start 72.630 61.500) (end 80.400 56.100) (width 0.22) (layer "F.Cu") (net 14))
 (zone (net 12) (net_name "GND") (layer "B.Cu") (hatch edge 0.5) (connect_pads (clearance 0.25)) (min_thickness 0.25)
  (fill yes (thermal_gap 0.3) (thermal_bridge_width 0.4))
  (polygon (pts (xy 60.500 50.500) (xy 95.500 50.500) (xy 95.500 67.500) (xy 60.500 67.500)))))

